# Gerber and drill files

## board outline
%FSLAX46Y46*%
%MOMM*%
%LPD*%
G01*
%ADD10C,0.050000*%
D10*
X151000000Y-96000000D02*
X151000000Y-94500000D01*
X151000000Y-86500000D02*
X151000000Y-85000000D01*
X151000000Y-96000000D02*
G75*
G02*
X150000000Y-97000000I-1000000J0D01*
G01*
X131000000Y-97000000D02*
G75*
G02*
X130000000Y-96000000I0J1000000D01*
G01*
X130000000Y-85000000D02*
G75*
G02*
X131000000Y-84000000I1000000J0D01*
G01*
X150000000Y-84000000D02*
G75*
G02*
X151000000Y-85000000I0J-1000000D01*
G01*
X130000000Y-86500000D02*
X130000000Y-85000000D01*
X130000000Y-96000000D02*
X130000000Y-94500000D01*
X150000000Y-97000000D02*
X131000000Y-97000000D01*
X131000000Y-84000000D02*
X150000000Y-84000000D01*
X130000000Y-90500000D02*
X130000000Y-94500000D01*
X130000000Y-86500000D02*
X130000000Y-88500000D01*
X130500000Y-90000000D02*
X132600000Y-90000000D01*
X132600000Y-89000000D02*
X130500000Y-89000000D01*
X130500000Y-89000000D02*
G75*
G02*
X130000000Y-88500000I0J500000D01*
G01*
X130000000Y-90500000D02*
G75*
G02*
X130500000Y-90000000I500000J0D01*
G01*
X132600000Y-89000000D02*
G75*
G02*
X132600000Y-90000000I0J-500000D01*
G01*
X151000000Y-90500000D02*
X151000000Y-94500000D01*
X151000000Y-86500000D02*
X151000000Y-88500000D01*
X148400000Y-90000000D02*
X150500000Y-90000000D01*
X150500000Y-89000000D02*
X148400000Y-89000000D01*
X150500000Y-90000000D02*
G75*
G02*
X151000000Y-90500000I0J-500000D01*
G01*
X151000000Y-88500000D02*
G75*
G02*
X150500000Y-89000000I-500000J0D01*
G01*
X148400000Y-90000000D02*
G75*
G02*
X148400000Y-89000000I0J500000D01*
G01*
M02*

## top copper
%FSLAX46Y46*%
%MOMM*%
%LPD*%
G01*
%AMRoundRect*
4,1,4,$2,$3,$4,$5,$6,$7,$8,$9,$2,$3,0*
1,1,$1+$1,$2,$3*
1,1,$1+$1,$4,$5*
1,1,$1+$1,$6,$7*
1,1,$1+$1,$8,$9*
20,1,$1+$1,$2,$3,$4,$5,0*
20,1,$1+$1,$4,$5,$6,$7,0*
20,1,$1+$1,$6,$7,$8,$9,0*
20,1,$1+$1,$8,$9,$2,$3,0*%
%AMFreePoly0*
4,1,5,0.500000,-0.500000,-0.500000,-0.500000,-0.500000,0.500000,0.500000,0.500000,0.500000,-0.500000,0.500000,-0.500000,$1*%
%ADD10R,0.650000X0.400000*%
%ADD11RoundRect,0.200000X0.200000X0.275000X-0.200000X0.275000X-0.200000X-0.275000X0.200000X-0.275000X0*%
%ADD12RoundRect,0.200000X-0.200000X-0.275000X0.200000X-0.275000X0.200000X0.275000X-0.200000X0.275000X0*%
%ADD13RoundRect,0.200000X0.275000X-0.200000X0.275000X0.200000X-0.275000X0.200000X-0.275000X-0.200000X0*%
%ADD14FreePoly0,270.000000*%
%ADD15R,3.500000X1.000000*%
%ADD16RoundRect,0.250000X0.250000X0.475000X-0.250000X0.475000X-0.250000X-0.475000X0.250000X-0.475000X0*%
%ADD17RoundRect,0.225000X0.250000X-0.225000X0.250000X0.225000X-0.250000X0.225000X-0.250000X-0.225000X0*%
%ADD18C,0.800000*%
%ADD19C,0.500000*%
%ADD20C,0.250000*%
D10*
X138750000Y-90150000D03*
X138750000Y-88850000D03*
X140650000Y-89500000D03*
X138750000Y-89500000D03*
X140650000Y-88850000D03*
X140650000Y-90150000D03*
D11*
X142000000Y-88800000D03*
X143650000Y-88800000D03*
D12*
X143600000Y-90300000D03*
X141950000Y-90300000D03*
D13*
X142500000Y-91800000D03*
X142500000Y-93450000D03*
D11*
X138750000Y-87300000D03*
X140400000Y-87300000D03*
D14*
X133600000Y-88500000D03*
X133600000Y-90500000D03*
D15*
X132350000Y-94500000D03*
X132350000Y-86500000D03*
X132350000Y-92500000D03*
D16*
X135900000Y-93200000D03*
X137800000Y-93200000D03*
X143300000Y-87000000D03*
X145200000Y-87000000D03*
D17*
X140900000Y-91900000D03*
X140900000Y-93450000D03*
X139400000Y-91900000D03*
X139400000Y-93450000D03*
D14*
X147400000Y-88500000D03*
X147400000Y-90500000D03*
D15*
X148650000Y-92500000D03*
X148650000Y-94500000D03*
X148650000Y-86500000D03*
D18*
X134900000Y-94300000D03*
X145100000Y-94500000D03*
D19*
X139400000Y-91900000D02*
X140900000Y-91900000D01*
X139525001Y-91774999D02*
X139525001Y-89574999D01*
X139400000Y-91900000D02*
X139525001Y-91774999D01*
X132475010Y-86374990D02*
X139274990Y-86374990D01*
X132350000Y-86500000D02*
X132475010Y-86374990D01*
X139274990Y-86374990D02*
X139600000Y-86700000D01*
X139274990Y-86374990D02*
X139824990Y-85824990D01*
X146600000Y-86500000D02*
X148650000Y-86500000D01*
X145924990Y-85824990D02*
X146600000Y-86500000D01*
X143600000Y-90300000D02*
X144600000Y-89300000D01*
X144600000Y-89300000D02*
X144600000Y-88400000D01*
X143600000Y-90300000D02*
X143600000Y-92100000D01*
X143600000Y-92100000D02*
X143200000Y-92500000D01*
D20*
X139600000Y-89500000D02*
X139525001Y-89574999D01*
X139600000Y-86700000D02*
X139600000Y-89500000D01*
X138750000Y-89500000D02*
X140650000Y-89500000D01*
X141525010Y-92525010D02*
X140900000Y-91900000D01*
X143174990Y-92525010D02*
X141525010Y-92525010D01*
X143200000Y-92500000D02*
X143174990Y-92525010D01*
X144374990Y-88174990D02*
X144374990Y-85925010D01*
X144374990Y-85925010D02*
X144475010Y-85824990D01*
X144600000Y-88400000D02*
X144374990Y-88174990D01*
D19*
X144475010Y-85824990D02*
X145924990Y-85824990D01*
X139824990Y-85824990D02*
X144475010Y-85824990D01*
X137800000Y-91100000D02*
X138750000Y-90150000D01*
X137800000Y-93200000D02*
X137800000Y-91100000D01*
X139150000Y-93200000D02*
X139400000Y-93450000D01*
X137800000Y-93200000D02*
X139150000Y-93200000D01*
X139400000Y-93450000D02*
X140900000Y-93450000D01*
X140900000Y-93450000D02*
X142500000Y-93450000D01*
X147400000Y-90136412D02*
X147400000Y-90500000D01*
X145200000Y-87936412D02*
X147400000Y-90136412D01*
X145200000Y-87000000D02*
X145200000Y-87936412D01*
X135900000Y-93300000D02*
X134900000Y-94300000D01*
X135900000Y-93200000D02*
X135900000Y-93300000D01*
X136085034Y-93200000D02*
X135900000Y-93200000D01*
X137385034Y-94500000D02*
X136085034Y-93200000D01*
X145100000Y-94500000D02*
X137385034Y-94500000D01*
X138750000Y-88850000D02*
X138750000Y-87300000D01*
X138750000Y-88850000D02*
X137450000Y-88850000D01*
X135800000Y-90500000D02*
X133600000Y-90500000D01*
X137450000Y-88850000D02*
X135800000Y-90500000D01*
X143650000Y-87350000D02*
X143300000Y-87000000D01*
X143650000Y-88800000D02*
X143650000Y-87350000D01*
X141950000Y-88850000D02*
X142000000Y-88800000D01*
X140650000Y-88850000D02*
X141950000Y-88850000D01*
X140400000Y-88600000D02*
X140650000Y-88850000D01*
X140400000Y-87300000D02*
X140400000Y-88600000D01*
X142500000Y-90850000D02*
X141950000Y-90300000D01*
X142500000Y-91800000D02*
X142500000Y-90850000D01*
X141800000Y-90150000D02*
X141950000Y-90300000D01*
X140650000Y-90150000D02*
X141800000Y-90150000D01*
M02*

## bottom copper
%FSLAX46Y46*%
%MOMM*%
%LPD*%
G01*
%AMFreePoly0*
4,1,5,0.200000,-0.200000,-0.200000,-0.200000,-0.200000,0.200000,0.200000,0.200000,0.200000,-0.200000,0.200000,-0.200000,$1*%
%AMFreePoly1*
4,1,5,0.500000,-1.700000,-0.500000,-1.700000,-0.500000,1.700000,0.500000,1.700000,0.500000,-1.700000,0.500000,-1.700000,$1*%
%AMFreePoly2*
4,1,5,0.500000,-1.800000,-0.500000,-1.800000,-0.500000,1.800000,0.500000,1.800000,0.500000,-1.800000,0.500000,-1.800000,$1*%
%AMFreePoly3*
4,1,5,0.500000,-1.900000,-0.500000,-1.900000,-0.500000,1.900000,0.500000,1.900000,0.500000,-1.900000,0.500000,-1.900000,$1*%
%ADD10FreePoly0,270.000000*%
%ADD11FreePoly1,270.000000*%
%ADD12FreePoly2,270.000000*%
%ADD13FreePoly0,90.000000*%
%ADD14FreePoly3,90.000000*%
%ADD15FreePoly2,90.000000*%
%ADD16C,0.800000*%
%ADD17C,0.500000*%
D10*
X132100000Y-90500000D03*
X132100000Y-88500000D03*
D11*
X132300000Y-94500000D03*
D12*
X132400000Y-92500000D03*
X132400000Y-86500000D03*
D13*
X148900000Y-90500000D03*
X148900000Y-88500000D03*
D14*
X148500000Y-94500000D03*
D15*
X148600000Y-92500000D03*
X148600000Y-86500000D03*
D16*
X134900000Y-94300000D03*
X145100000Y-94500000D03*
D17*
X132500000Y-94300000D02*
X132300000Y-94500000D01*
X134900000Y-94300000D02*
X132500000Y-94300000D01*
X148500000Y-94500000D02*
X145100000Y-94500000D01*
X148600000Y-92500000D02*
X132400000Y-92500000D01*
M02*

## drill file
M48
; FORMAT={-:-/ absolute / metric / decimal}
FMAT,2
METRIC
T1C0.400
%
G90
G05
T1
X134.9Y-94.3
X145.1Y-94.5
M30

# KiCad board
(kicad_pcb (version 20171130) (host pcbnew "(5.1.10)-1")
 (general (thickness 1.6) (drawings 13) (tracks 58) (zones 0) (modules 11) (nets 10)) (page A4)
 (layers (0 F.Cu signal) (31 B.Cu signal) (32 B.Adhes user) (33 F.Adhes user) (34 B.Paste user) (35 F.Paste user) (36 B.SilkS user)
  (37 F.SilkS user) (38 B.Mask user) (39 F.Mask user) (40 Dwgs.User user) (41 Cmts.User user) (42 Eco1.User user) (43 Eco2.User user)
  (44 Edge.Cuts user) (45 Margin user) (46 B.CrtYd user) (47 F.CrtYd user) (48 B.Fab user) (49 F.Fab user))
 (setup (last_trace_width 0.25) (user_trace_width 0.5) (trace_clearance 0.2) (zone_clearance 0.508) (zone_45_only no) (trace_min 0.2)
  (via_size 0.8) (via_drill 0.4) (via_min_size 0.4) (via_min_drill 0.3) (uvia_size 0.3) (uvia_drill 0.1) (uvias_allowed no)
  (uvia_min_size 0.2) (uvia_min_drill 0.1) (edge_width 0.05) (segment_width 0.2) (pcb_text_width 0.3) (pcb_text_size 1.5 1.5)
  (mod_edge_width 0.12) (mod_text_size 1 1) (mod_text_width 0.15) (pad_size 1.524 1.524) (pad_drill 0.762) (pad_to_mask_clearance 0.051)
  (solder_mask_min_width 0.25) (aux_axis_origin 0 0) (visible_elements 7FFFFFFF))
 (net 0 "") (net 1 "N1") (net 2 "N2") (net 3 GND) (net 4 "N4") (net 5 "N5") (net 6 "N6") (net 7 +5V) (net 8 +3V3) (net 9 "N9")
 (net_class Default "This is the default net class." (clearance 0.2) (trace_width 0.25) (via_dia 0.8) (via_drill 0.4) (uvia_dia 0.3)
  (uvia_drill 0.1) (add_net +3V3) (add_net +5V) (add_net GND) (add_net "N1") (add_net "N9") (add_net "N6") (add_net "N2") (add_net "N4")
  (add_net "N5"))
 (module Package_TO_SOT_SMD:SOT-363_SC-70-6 (layer F.Cu) (at 139.7 89.5 180)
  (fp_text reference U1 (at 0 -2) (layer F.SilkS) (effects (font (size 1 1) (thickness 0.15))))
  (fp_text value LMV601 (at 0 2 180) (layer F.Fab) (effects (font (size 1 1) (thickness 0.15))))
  (pad 6 smd rect (at 0.95 -0.65 180) (size 0.65 0.4) (layers F.Cu F.Paste F.Mask) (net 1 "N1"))
  (pad 4 smd rect (at 0.95 0.65 180) (size 0.65 0.4) (layers F.Cu F.Paste F.Mask) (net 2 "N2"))
  (pad 2 smd rect (at -0.95 0 180) (size 0.65 0.4) (layers F.Cu F.Paste F.Mask) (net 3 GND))
  (pad 5 smd rect (at 0.95 0 180) (size 0.65 0.4) (layers F.Cu F.Paste F.Mask) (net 3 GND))
  (pad 3 smd rect (at -0.95 0.65 180) (size 0.65 0.4) (layers F.Cu F.Paste F.Mask) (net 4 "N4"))
  (pad 1 smd rect (at -0.95 -0.65 180) (size 0.65 0.4) (layers F.Cu F.Paste F.Mask) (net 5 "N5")))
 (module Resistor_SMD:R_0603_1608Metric (layer F.Cu) (at 142.825 88.8 180)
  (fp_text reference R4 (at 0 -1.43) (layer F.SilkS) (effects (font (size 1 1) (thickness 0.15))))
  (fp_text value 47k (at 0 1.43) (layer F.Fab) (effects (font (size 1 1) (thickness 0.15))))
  (pad 2 smd roundrect (at 0.825 0 180) (size 0.8 0.95) (layers F.Cu F.Paste F.Mask) (roundrect_rratio 0.25) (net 4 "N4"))
  (pad 1 smd roundrect (at -0.825 0 180) (size 0.8 0.95) (layers F.Cu F.Paste F.Mask) (roundrect_rratio 0.25) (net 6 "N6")))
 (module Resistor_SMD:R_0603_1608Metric (layer F.Cu) (at 142.775 90.3)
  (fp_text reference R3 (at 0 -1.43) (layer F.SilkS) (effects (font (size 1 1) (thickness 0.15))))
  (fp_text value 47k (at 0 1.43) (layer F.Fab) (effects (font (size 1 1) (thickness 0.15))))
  (pad 2 smd roundrect (at 0.825 0) (size 0.8 0.95) (layers F.Cu F.Paste F.Mask) (roundrect_rratio 0.25) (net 3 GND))
  (pad 1 smd roundrect (at -0.825 0) (size 0.8 0.95) (layers F.Cu F.Paste F.Mask) (roundrect_rratio 0.25) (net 5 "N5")))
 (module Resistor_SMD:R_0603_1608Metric (layer F.Cu) (at 142.5 92.625 90)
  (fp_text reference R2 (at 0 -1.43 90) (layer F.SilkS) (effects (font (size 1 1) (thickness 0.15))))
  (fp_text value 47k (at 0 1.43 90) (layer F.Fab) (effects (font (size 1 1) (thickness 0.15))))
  (pad 2 smd roundrect (at 0.825 0 90) (size 0.8 0.95) (layers F.Cu F.Paste F.Mask) (roundrect_rratio 0.25) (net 5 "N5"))
  (pad 1 smd roundrect (at -0.825 0 90) (size 0.8 0.95) (layers F.Cu F.Paste F.Mask) (roundrect_rratio 0.25) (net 1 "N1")))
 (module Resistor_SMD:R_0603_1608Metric (layer F.Cu) (at 139.575 87.3 180)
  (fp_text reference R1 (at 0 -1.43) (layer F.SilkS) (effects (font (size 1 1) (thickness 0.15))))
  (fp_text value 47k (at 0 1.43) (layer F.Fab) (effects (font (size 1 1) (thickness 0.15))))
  (pad 2 smd roundrect (at 0.825 0 180) (size 0.8 0.95) (layers F.Cu F.Paste F.Mask) (roundrect_rratio 0.25) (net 2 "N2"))
  (pad 1 smd roundrect (at -0.825 0 180) (size 0.8 0.95) (layers F.Cu F.Paste F.Mask) (roundrect_rratio 0.25) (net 4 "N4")))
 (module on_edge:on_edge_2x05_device (layer F.Cu) (at 130 90.5 270)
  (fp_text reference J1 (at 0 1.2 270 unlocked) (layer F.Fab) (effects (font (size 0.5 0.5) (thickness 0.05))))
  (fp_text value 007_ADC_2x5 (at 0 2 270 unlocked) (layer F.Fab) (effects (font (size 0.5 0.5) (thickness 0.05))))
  (fp_line (start 0 0) (end 4 0) (layer Edge.Cuts) (width 0.05))
  (fp_line (start -4 0) (end -2 0) (layer Edge.Cuts) (width 0.05))
  (fp_line (start -0.5 -0.5) (end -0.5 -2.6) (layer Edge.Cuts) (width 0.05))
  (fp_line (start -1.5 -2.6) (end -1.5 -0.5) (layer Edge.Cuts) (width 0.05))
  (fp_arc (start -2 -0.5) (end -2 0) (angle -90) (layer Edge.Cuts) (width 0.05))
  (fp_arc (start 0 -0.5) (end -0.5 -0.5) (angle -90) (layer Edge.Cuts) (width 0.05))
  (fp_arc (start -1 -2.6) (end -0.5 -2.6) (angle -180) (layer Edge.Cuts) (width 0.05))
  (pad 2 smd custom (at -2 -3.6 270) (size 1 1) (layers F.Cu F.Mask) (zone_connect 0) (options (clearance outline) (anchor rect))
   (primitives))
  (pad 3 smd custom (at 0 -3.6 270) (size 1 1) (layers F.Cu F.Mask) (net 2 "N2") (zone_connect 0)
   (options (clearance outline) (anchor rect)) (primitives))
  (pad 8 smd custom (at 0 -2.1 270) (size 0.4 0.4) (layers B.Cu B.Mask) (zone_connect 0) (options (clearance outline) (anchor rect))
   (primitives))
  (pad 7 smd custom (at -2 -2.1 270) (size 0.4 0.4) (layers B.Cu B.Mask) (zone_connect 0) (options (clearance outline) (anchor rect))
   (primitives))
  (pad 10 smd custom (at 4 -2.3 270) (size 1 3.4) (layers B.Cu B.Mask) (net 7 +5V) (zone_connect 0)
   (options (clearance outline) (anchor rect)) (primitives))
  (pad 9 smd custom (at 2 -2.4 270) (size 1 3.6) (layers B.Cu B.Mask) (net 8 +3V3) (zone_connect 0)
   (options (clearance outline) (anchor rect)) (primitives))
  (pad 6 smd custom (at -4 -2.4 270) (size 1 3.6) (layers B.Cu B.Mask) (zone_connect 0) (options (clearance outline) (anchor rect))
   (primitives))
  (pad 5 smd rect (at 4 -2.35 90) (size 1 3.5) (layers F.Cu F.Mask) (zone_connect 0))
  (pad 1 smd rect (at -4 -2.35 90) (size 1 3.5) (layers F.Cu F.Mask) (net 3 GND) (zone_connect 0))
  (pad 4 smd rect (at 2 -2.35 90) (size 1 3.5) (layers F.Cu F.Mask) (zone_connect 0)))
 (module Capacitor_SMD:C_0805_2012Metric (layer F.Cu) (at 136.85 93.2 180)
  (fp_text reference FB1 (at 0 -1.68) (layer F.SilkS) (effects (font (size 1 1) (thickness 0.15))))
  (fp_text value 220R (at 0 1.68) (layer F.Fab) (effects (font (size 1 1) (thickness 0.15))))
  (pad 2 smd roundrect (at 0.95 0 180) (size 1 1.45) (layers F.Cu F.Paste F.Mask) (roundrect_rratio 0.25) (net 7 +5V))
  (pad 1 smd roundrect (at -0.95 0 180) (size 1 1.45) (layers F.Cu F.Paste F.Mask) (roundrect_rratio 0.25) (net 1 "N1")))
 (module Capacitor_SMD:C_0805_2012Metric (layer F.Cu) (at 144.25 87 180)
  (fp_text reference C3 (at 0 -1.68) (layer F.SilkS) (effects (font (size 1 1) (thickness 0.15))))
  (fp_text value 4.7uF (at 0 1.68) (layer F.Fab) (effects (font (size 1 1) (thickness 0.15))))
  (pad 2 smd roundrect (at 0.95 0 180) (size 1 1.45) (layers F.Cu F.Paste F.Mask) (roundrect_rratio 0.25) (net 6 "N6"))
  (pad 1 smd roundrect (at -0.95 0 180) (size 1 1.45) (layers F.Cu F.Paste F.Mask) (roundrect_rratio 0.25) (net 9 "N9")))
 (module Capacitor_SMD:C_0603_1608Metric (layer F.Cu) (at 140.9 92.675 90)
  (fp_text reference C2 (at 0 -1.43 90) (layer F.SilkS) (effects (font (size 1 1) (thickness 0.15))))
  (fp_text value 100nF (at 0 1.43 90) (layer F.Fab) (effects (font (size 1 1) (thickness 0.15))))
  (pad 2 smd roundrect (at 0.775 0 90) (size 0.9 0.95) (layers F.Cu F.Paste F.Mask) (roundrect_rratio 0.25) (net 3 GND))
  (pad 1 smd roundrect (at -0.775 0 90) (size 0.9 0.95) (layers F.Cu F.Paste F.Mask) (roundrect_rratio 0.25) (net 1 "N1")))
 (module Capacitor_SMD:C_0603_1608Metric (layer F.Cu) (at 139.4 92.675 90)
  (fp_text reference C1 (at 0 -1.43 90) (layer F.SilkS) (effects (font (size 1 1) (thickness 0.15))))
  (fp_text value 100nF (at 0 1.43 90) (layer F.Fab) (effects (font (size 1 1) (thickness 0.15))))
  (pad 2 smd roundrect (at 0.775 0 90) (size 0.9 0.95) (layers F.Cu F.Paste F.Mask) (roundrect_rratio 0.25) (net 3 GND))
  (pad 1 smd roundrect (at -0.775 0 90) (size 0.9 0.95) (layers F.Cu F.Paste F.Mask) (roundrect_rratio 0.25) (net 1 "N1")))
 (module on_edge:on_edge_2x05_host (layer F.Cu) (at 151 90.5 270)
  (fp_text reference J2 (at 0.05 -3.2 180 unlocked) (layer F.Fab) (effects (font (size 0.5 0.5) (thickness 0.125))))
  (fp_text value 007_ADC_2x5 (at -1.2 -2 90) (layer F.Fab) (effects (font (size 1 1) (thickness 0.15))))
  (fp_line (start 0 0) (end 4 0) (layer Edge.Cuts) (width 0.05))
  (fp_line (start -4 0) (end -2 0) (layer Edge.Cuts) (width 0.05))
  (fp_line (start -0.5 2.6) (end -0.5 0.5) (layer Edge.Cuts) (width 0.05))
  (fp_line (start -1.5 0.5) (end -1.5 2.6) (layer Edge.Cuts) (width 0.05))
  (fp_arc (start 0 0.5) (end 0 0) (angle -90) (layer Edge.Cuts) (width 0.05))
  (fp_arc (start -2 0.5) (end -1.5 0.5) (angle -90) (layer Edge.Cuts) (width 0.05))
  (fp_arc (start -1 2.6) (end -1.5 2.6) (angle -180) (layer Edge.Cuts) (width 0.05))
  (pad 2 smd custom (at -2 3.6 270) (size 1 1) (layers F.Cu F.Mask) (zone_connect 0) (options (clearance outline) (anchor rect))
   (primitives))
  (pad 3 smd custom (at 0 3.6 270) (size 1 1) (layers F.Cu F.Mask) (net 9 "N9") (zone_connect 0) (options (clearance outline) (anchor rect))
   (primitives))
  (pad 8 smd custom (at 0 2.1 90) (size 0.4 0.4) (layers B.Cu B.Mask) (zone_connect 0) (options (clearance outline) (anchor rect))
   (primitives))
  (pad 7 smd custom (at -2 2.1 90) (size 0.4 0.4) (layers B.Cu B.Mask) (zone_connect 0) (options (clearance outline) (anchor rect))
   (primitives))
  (pad 4 smd rect (at 2 2.35 270) (size 1 3.5) (layers F.Cu F.Mask) (zone_connect 0))
  (pad 10 smd custom (at 4 2.5 90) (size 1 3.8) (layers B.Cu B.Mask) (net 7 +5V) (zone_connect 0)
   (options (clearance outline) (anchor rect)) (primitives))
  (pad 9 smd custom (at 2 2.4 90) (size 1 3.6) (layers B.Cu B.Mask) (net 8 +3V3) (zone_connect 0)
   (options (clearance outline) (anchor rect)) (primitives))
  (pad 6 smd custom (at -4 2.4 90) (size 1 3.6) (layers B.Cu B.Mask) (zone_connect 0) (options (clearance outline) (anchor rect))
   (primitives))
  (pad 5 smd rect (at 4 2.35 270) (size 1 3.5) (layers F.Cu F.Mask) (zone_connect 0))
  (pad 1 smd rect (at -4 2.35 270) (size 1 3.5) (layers F.Cu F.Mask) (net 3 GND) (zone_connect 0)))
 (gr_line (start 151 96) (end 151 94.5) (layer Edge.Cuts) (width 0.05))
 (gr_line (start 151 86.5) (end 151 85) (layer Edge.Cuts) (width 0.05))
 (gr_arc (start 150 96) (end 150 97) (angle -90) (layer Edge.Cuts) (width 0.05))
 (gr_arc (start 131 96) (end 130 96) (angle -90) (layer Edge.Cuts) (width 0.05))
 (gr_arc (start 131 85) (end 131 84) (angle -90) (layer Edge.Cuts) (width 0.05))
 (gr_arc (start 150 85) (end 151 85) (angle -90) (layer Edge.Cuts) (width 0.05))
 (gr_line (start 130 86.5) (end 130 85) (layer Edge.Cuts) (width 0.05))
 (gr_line (start 130 96) (end 130 94.5) (layer Edge.Cuts) (width 0.05))
 (gr_line (start 150 97) (end 131 97) (layer Edge.Cuts) (width 0.05))
 (gr_line (start 131 84) (end 150 84) (layer Edge.Cuts) (width 0.05))
 (segment (start 139.4 91.9) (end 140.9 91.9) (width 0.5) (layer F.Cu) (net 3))
 (segment (start 139.525001 91.774999) (end 139.525001 89.574999) (width 0.5) (layer F.Cu) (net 3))
 (segment (start 139.4 91.9) (end 139.525001 91.774999) (width 0.5) (layer F.Cu) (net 3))
 (segment (start 132.47501 86.37499) (end 139.27499 86.37499) (width 0.5) (layer F.Cu) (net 3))
 (segment (start 132.35 86.5) (end 132.47501 86.37499) (width 0.5) (layer F.Cu) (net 3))
 (segment (start 139.27499 86.37499) (end 139.6 86.7) (width 0.5) (layer F.Cu) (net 3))
 (segment (start 139.27499 86.37499) (end 139.82499 85.82499) (width 0.5) (layer F.Cu) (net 3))
 (segment (start 146.6 86.5) (end 148.65 86.5) (width 0.5) (layer F.Cu) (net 3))
 (segment (start 145.92499 85.82499) (end 146.6 86.5) (width 0.5) (layer F.Cu) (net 3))
 (segment (start 143.6 90.3) (end 144.6 89.3) (width 0.5) (layer F.Cu) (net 3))
 (segment (start 144.6 89.3) (end 144.6 88.4) (width 0.5) (layer F.Cu) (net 3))
 (segment (start 143.6 90.3) (end 143.6 92.1) (width 0.5) (layer F.Cu) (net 3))
 (segment (start 143.6 92.1) (end 143.2 92.5) (width 0.5) (layer F.Cu) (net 3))
 (segment (start 139.6 89.5) (end 139.525001 89.574999) (width 0.25) (layer F.Cu) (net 3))
 (segment (start 139.6 86.7) (end 139.6 89.5) (width 0.25) (layer F.Cu) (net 3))
 (segment (start 138.75 89.5) (end 140.65 89.5) (width 0.25) (layer F.Cu) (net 3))
 (segment (start 141.52501 92.52501) (end 140.9 91.9) (width 0.25) (layer F.Cu) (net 3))
 (segment (start 143.17499 92.52501) (end 141.52501 92.52501) (width 0.25) (layer F.Cu) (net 3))
 (segment (start 143.2 92.5) (end 143.17499 92.52501) (width 0.25) (layer F.Cu) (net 3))
 (segment (start 144.37499 88.17499) (end 144.37499 85.92501) (width 0.25) (layer F.Cu) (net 3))
 (segment (start 144.37499 85.92501) (end 144.47501 85.82499) (width 0.25) (layer F.Cu) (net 3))
 (segment (start 144.6 88.4) (end 144.37499 88.17499) (width 0.25) (layer F.Cu) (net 3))
 (segment (start 144.47501 85.82499) (end 145.92499 85.82499) (width 0.5) (layer F.Cu) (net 3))
 (segment (start 139.82499 85.82499) (end 144.47501 85.82499) (width 0.5) (layer F.Cu) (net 3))
 (segment (start 137.8 91.1) (end 138.75 90.15) (width 0.5) (layer F.Cu) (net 1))
 (segment (start 137.8 93.2) (end 137.8 91.1) (width 0.5) (layer F.Cu) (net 1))
 (segment (start 139.15 93.2) (end 139.4 93.45) (width 0.5) (layer F.Cu) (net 1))
 (segment (start 137.8 93.2) (end 139.15 93.2) (width 0.5) (layer F.Cu) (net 1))
 (segment (start 139.4 93.45) (end 140.9 93.45) (width 0.5) (layer F.Cu) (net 1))
 (segment (start 140.9 93.45) (end 142.5 93.45) (width 0.5) (layer F.Cu) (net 1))
 (segment (start 147.4 90.136412) (end 147.4 90.5) (width 0.5) (layer F.Cu) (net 9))
 (segment (start 145.2 87.936412) (end 147.4 90.136412) (width 0.5) (layer F.Cu) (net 9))
 (segment (start 145.2 87) (end 145.2 87.936412) (width 0.5) (layer F.Cu) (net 9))
 (via (at 134.9 94.3) (size 0.8) (drill 0.4) (layers F.Cu B.Cu) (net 7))
 (segment (start 135.9 93.3) (end 134.9 94.3) (width 0.5) (layer F.Cu) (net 7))
 (segment (start 135.9 93.2) (end 135.9 93.3) (width 0.5) (layer F.Cu) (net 7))
 (segment (start 132.5 94.3) (end 132.3 94.5) (width 0.5) (layer B.Cu) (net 7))
 (segment (start 134.9 94.3) (end 132.5 94.3) (width 0.5) (layer B.Cu) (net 7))
 (via (at 145.1 94.5) (size 0.8) (drill 0.4) (layers F.Cu B.Cu) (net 7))
 (segment (start 148.5 94.5) (end 145.1 94.5) (width 0.5) (layer B.Cu) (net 7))
 (segment (start 136.085034 93.2) (end 135.9 93.2) (width 0.5) (layer F.Cu) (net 7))
 (segment (start 137.385034 94.5) (end 136.085034 93.2) (width 0.5) (layer F.Cu) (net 7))
 (segment (start 145.1 94.5) (end 137.385034 94.5) (width 0.5) (layer F.Cu) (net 7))
 (segment (start 138.75 88.85) (end 138.75 87.3) (width 0.5) (layer F.Cu) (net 2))
 (segment (start 138.75 88.85) (end 137.45 88.85) (width 0.5) (layer F.Cu) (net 2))
 (segment (start 135.8 90.5) (end 133.6 90.5) (width 0.5) (layer F.Cu) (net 2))
 (segment (start 137.45 88.85) (end 135.8 90.5) (width 0.5) (layer F.Cu) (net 2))
 (segment (start 148.6 92.5) (end 132.4 92.5) (width 0.5) (layer B.Cu) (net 8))
 (segment (start 143.65 87.35) (end 143.3 87) (width 0.5) (layer F.Cu) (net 6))
 (segment (start 143.65 88.8) (end 143.65 87.35) (width 0.5) (layer F.Cu) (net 6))
 (segment (start 141.95 88.85) (end 142 88.8) (width 0.5) (layer F.Cu) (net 4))
 (segment (start 140.65 88.85) (end 141.95 88.85) (width 0.5) (layer F.Cu) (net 4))
 (segment (start 140.4 88.6) (end 140.65 88.85) (width 0.5) (layer F.Cu) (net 4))
 (segment (start 140.4 87.3) (end 140.4 88.6) (width 0.5) (layer F.Cu) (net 4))
 (segment (start 142.5 90.85) (end 141.95 90.3) (width 0.5) (layer F.Cu) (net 5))
 (segment (start 142.5 91.8) (end 142.5 90.85) (width 0.5) (layer F.Cu) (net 5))
 (segment (start 141.8 90.15) (end 141.95 90.3) (width 0.5) (layer F.Cu) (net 5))
 (segment (start 140.65 90.15) (end 141.8 90.15) (width 0.5) (layer F.Cu) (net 5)))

